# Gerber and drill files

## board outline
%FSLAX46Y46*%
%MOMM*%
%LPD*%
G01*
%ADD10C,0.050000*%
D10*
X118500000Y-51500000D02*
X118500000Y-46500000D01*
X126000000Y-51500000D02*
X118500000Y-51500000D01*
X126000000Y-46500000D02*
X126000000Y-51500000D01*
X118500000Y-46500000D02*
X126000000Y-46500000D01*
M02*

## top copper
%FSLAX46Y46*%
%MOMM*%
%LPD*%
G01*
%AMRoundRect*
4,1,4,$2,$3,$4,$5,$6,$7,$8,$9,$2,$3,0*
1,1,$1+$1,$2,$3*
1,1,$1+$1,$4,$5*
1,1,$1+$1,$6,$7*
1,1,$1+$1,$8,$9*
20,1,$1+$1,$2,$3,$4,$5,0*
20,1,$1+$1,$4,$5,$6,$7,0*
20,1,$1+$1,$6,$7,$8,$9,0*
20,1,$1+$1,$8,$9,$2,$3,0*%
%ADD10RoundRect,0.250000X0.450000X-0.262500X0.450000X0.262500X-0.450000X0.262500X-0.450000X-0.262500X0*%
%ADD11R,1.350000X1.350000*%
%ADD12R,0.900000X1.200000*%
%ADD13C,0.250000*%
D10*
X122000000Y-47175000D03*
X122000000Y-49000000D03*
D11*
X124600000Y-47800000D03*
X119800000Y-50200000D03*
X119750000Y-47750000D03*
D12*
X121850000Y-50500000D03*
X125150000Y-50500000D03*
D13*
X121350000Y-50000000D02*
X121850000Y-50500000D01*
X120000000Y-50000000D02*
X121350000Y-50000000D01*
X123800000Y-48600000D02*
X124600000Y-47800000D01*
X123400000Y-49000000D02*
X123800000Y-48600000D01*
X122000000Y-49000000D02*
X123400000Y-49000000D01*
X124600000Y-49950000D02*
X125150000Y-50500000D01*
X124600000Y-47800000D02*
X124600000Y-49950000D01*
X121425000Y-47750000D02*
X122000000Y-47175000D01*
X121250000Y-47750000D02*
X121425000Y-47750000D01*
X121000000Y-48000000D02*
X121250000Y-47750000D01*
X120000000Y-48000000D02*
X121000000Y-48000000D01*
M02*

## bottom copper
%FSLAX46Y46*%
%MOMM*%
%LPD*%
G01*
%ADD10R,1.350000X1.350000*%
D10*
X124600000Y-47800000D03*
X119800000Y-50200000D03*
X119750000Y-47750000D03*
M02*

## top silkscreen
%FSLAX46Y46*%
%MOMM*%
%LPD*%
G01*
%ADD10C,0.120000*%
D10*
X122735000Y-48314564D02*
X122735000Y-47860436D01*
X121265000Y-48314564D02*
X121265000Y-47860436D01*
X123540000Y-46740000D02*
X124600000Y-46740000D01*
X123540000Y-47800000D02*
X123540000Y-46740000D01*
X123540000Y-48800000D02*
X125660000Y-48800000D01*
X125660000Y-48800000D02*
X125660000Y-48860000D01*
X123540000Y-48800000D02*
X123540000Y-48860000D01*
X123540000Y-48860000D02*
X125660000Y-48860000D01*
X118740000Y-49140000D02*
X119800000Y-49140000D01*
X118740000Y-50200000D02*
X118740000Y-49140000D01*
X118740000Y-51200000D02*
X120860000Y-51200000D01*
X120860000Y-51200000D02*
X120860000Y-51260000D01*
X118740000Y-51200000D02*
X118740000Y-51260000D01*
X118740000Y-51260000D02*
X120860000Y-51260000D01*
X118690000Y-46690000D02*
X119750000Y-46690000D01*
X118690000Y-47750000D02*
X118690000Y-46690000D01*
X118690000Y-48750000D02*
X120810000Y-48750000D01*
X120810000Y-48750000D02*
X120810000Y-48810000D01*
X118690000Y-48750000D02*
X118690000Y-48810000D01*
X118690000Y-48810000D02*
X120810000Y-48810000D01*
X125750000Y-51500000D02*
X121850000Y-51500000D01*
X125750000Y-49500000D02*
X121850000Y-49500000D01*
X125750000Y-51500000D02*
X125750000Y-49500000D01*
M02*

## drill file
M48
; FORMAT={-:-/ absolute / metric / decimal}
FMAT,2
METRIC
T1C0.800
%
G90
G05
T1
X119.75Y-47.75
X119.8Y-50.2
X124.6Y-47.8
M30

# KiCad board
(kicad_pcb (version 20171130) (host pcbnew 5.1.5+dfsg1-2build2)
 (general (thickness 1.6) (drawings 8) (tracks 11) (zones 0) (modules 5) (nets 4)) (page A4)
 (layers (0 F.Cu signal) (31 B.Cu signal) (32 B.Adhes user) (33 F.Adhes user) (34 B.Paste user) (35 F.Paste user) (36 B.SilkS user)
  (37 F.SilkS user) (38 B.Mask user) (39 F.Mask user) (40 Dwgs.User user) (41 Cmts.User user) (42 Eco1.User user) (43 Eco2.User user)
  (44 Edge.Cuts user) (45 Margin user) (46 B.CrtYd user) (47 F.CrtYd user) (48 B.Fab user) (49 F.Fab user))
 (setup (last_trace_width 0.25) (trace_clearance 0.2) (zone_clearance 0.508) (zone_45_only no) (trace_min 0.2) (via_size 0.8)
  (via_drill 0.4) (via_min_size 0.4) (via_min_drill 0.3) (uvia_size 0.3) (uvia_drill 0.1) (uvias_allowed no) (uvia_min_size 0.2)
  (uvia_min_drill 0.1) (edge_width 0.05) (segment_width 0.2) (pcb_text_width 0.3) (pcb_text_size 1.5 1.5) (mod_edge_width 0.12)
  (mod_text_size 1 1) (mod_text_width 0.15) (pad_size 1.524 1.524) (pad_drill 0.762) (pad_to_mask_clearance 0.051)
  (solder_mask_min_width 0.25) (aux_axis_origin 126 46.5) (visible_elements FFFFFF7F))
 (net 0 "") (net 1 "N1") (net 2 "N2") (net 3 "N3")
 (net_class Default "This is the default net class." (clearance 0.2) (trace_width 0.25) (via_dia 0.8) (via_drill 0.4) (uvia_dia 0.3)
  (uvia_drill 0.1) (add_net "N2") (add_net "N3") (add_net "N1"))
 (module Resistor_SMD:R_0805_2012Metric (layer F.Cu) (at 122 48.0875 90)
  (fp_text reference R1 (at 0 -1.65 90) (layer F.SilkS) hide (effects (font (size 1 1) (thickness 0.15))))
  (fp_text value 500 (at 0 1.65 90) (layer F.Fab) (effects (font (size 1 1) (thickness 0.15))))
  (fp_line (start -0.227064 0.735) (end 0.227064 0.735) (layer F.SilkS) (width 0.12))
  (fp_line (start -0.227064 -0.735) (end 0.227064 -0.735) (layer F.SilkS) (width 0.12))
  (pad 2 smd roundrect (at 0.9125 0 90) (size 1.025 1.4) (layers F.Cu F.Paste F.Mask) (roundrect_rratio 0.243902) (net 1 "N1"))
  (pad 1 smd roundrect (at -0.9125 0 90) (size 1.025 1.4) (layers F.Cu F.Paste F.Mask) (roundrect_rratio 0.243902) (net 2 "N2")))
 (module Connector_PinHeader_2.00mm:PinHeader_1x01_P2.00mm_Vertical (layer F.Cu) (at 124.6 47.8)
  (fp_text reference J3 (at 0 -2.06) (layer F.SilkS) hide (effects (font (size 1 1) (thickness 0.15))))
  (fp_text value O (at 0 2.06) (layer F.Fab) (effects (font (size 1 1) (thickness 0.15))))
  (fp_line (start -1.06 -1.06) (end 0 -1.06) (layer F.SilkS) (width 0.12))
  (fp_line (start -1.06 0) (end -1.06 -1.06) (layer F.SilkS) (width 0.12))
  (fp_line (start -1.06 1) (end 1.06 1) (layer F.SilkS) (width 0.12))
  (fp_line (start 1.06 1) (end 1.06 1.06) (layer F.SilkS) (width 0.12))
  (fp_line (start -1.06 1) (end -1.06 1.06) (layer F.SilkS) (width 0.12))
  (fp_line (start -1.06 1.06) (end 1.06 1.06) (layer F.SilkS) (width 0.12))
  (pad 1 thru_hole rect (at 0 0) (size 1.35 1.35) (drill 0.8) (layers *.Cu *.Mask) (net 2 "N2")))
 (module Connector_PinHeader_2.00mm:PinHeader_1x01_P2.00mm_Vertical (layer F.Cu) (at 119.8 50.2)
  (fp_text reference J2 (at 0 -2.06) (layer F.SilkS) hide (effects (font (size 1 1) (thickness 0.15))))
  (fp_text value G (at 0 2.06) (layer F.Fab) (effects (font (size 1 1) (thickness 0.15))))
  (fp_line (start -1.06 -1.06) (end 0 -1.06) (layer F.SilkS) (width 0.12))
  (fp_line (start -1.06 0) (end -1.06 -1.06) (layer F.SilkS) (width 0.12))
  (fp_line (start -1.06 1) (end 1.06 1) (layer F.SilkS) (width 0.12))
  (fp_line (start 1.06 1) (end 1.06 1.06) (layer F.SilkS) (width 0.12))
  (fp_line (start -1.06 1) (end -1.06 1.06) (layer F.SilkS) (width 0.12))
  (fp_line (start -1.06 1.06) (end 1.06 1.06) (layer F.SilkS) (width 0.12))
  (pad 1 thru_hole rect (at 0 0) (size 1.35 1.35) (drill 0.8) (layers *.Cu *.Mask) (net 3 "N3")))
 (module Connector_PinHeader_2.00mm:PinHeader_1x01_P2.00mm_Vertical (layer F.Cu) (at 119.75 47.75)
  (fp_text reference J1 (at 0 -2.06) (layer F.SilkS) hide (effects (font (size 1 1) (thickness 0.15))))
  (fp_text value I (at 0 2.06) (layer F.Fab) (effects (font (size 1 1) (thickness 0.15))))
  (fp_line (start -1.06 -1.06) (end 0 -1.06) (layer F.SilkS) (width 0.12))
  (fp_line (start -1.06 0) (end -1.06 -1.06) (layer F.SilkS) (width 0.12))
  (fp_line (start -1.06 1) (end 1.06 1) (layer F.SilkS) (width 0.12))
  (fp_line (start 1.06 1) (end 1.06 1.06) (layer F.SilkS) (width 0.12))
  (fp_line (start -1.06 1) (end -1.06 1.06) (layer F.SilkS) (width 0.12))
  (fp_line (start -1.06 1.06) (end 1.06 1.06) (layer F.SilkS) (width 0.12))
  (pad 1 thru_hole rect (at 0 0) (size 1.35 1.35) (drill 0.8) (layers *.Cu *.Mask) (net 1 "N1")))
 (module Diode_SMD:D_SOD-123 (layer F.Cu) (at 123.5 50.5 180)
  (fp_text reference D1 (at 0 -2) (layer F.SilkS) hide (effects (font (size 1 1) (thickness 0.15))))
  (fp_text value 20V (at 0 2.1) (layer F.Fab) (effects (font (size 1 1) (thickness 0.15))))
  (fp_line (start -2.25 -1) (end 1.65 -1) (layer F.SilkS) (width 0.12))
  (fp_line (start -2.25 1) (end 1.65 1) (layer F.SilkS) (width 0.12))
  (fp_line (start -2.25 -1) (end -2.25 1) (layer F.SilkS) (width 0.12))
  (pad 2 smd rect (at 1.65 0 180) (size 0.9 1.2) (layers F.Cu F.Paste F.Mask) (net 3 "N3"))
  (pad 1 smd rect (at -1.65 0 180) (size 0.9 1.2) (layers F.Cu F.Paste F.Mask) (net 2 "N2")))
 (gr_line (start 118.5 51.5) (end 118.5 46.5) (layer Edge.Cuts) (width 0.05))
 (gr_line (start 126 51.5) (end 118.5 51.5) (layer Edge.Cuts) (width 0.05))
 (gr_line (start 126 46.5) (end 126 51.5) (layer Edge.Cuts) (width 0.05))
 (gr_line (start 118.5 46.5) (end 126 46.5) (layer Edge.Cuts) (width 0.05))
 (segment (start 121.35 50) (end 121.85 50.5) (width 0.25) (layer F.Cu) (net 3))
 (segment (start 120 50) (end 121.35 50) (width 0.25) (layer F.Cu) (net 3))
 (segment (start 123.8 48.6) (end 124.6 47.8) (width 0.25) (layer F.Cu) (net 2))
 (segment (start 123.4 49) (end 123.8 48.6) (width 0.25) (layer F.Cu) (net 2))
 (segment (start 122 49) (end 123.4 49) (width 0.25) (layer F.Cu) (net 2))
 (segment (start 124.6 49.95) (end 125.15 50.5) (width 0.25) (layer F.Cu) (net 2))
 (segment (start 124.6 47.8) (end 124.6 49.95) (width 0.25) (layer F.Cu) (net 2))
 (segment (start 121.425 47.75) (end 122 47.175) (width 0.25) (layer F.Cu) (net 1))
 (segment (start 121.25 47.75) (end 121.425 47.75) (width 0.25) (layer F.Cu) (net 1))
 (segment (start 121 48) (end 121.25 47.75) (width 0.25) (layer F.Cu) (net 1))
 (segment (start 120 48) (end 121 48) (width 0.25) (layer F.Cu) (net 1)))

